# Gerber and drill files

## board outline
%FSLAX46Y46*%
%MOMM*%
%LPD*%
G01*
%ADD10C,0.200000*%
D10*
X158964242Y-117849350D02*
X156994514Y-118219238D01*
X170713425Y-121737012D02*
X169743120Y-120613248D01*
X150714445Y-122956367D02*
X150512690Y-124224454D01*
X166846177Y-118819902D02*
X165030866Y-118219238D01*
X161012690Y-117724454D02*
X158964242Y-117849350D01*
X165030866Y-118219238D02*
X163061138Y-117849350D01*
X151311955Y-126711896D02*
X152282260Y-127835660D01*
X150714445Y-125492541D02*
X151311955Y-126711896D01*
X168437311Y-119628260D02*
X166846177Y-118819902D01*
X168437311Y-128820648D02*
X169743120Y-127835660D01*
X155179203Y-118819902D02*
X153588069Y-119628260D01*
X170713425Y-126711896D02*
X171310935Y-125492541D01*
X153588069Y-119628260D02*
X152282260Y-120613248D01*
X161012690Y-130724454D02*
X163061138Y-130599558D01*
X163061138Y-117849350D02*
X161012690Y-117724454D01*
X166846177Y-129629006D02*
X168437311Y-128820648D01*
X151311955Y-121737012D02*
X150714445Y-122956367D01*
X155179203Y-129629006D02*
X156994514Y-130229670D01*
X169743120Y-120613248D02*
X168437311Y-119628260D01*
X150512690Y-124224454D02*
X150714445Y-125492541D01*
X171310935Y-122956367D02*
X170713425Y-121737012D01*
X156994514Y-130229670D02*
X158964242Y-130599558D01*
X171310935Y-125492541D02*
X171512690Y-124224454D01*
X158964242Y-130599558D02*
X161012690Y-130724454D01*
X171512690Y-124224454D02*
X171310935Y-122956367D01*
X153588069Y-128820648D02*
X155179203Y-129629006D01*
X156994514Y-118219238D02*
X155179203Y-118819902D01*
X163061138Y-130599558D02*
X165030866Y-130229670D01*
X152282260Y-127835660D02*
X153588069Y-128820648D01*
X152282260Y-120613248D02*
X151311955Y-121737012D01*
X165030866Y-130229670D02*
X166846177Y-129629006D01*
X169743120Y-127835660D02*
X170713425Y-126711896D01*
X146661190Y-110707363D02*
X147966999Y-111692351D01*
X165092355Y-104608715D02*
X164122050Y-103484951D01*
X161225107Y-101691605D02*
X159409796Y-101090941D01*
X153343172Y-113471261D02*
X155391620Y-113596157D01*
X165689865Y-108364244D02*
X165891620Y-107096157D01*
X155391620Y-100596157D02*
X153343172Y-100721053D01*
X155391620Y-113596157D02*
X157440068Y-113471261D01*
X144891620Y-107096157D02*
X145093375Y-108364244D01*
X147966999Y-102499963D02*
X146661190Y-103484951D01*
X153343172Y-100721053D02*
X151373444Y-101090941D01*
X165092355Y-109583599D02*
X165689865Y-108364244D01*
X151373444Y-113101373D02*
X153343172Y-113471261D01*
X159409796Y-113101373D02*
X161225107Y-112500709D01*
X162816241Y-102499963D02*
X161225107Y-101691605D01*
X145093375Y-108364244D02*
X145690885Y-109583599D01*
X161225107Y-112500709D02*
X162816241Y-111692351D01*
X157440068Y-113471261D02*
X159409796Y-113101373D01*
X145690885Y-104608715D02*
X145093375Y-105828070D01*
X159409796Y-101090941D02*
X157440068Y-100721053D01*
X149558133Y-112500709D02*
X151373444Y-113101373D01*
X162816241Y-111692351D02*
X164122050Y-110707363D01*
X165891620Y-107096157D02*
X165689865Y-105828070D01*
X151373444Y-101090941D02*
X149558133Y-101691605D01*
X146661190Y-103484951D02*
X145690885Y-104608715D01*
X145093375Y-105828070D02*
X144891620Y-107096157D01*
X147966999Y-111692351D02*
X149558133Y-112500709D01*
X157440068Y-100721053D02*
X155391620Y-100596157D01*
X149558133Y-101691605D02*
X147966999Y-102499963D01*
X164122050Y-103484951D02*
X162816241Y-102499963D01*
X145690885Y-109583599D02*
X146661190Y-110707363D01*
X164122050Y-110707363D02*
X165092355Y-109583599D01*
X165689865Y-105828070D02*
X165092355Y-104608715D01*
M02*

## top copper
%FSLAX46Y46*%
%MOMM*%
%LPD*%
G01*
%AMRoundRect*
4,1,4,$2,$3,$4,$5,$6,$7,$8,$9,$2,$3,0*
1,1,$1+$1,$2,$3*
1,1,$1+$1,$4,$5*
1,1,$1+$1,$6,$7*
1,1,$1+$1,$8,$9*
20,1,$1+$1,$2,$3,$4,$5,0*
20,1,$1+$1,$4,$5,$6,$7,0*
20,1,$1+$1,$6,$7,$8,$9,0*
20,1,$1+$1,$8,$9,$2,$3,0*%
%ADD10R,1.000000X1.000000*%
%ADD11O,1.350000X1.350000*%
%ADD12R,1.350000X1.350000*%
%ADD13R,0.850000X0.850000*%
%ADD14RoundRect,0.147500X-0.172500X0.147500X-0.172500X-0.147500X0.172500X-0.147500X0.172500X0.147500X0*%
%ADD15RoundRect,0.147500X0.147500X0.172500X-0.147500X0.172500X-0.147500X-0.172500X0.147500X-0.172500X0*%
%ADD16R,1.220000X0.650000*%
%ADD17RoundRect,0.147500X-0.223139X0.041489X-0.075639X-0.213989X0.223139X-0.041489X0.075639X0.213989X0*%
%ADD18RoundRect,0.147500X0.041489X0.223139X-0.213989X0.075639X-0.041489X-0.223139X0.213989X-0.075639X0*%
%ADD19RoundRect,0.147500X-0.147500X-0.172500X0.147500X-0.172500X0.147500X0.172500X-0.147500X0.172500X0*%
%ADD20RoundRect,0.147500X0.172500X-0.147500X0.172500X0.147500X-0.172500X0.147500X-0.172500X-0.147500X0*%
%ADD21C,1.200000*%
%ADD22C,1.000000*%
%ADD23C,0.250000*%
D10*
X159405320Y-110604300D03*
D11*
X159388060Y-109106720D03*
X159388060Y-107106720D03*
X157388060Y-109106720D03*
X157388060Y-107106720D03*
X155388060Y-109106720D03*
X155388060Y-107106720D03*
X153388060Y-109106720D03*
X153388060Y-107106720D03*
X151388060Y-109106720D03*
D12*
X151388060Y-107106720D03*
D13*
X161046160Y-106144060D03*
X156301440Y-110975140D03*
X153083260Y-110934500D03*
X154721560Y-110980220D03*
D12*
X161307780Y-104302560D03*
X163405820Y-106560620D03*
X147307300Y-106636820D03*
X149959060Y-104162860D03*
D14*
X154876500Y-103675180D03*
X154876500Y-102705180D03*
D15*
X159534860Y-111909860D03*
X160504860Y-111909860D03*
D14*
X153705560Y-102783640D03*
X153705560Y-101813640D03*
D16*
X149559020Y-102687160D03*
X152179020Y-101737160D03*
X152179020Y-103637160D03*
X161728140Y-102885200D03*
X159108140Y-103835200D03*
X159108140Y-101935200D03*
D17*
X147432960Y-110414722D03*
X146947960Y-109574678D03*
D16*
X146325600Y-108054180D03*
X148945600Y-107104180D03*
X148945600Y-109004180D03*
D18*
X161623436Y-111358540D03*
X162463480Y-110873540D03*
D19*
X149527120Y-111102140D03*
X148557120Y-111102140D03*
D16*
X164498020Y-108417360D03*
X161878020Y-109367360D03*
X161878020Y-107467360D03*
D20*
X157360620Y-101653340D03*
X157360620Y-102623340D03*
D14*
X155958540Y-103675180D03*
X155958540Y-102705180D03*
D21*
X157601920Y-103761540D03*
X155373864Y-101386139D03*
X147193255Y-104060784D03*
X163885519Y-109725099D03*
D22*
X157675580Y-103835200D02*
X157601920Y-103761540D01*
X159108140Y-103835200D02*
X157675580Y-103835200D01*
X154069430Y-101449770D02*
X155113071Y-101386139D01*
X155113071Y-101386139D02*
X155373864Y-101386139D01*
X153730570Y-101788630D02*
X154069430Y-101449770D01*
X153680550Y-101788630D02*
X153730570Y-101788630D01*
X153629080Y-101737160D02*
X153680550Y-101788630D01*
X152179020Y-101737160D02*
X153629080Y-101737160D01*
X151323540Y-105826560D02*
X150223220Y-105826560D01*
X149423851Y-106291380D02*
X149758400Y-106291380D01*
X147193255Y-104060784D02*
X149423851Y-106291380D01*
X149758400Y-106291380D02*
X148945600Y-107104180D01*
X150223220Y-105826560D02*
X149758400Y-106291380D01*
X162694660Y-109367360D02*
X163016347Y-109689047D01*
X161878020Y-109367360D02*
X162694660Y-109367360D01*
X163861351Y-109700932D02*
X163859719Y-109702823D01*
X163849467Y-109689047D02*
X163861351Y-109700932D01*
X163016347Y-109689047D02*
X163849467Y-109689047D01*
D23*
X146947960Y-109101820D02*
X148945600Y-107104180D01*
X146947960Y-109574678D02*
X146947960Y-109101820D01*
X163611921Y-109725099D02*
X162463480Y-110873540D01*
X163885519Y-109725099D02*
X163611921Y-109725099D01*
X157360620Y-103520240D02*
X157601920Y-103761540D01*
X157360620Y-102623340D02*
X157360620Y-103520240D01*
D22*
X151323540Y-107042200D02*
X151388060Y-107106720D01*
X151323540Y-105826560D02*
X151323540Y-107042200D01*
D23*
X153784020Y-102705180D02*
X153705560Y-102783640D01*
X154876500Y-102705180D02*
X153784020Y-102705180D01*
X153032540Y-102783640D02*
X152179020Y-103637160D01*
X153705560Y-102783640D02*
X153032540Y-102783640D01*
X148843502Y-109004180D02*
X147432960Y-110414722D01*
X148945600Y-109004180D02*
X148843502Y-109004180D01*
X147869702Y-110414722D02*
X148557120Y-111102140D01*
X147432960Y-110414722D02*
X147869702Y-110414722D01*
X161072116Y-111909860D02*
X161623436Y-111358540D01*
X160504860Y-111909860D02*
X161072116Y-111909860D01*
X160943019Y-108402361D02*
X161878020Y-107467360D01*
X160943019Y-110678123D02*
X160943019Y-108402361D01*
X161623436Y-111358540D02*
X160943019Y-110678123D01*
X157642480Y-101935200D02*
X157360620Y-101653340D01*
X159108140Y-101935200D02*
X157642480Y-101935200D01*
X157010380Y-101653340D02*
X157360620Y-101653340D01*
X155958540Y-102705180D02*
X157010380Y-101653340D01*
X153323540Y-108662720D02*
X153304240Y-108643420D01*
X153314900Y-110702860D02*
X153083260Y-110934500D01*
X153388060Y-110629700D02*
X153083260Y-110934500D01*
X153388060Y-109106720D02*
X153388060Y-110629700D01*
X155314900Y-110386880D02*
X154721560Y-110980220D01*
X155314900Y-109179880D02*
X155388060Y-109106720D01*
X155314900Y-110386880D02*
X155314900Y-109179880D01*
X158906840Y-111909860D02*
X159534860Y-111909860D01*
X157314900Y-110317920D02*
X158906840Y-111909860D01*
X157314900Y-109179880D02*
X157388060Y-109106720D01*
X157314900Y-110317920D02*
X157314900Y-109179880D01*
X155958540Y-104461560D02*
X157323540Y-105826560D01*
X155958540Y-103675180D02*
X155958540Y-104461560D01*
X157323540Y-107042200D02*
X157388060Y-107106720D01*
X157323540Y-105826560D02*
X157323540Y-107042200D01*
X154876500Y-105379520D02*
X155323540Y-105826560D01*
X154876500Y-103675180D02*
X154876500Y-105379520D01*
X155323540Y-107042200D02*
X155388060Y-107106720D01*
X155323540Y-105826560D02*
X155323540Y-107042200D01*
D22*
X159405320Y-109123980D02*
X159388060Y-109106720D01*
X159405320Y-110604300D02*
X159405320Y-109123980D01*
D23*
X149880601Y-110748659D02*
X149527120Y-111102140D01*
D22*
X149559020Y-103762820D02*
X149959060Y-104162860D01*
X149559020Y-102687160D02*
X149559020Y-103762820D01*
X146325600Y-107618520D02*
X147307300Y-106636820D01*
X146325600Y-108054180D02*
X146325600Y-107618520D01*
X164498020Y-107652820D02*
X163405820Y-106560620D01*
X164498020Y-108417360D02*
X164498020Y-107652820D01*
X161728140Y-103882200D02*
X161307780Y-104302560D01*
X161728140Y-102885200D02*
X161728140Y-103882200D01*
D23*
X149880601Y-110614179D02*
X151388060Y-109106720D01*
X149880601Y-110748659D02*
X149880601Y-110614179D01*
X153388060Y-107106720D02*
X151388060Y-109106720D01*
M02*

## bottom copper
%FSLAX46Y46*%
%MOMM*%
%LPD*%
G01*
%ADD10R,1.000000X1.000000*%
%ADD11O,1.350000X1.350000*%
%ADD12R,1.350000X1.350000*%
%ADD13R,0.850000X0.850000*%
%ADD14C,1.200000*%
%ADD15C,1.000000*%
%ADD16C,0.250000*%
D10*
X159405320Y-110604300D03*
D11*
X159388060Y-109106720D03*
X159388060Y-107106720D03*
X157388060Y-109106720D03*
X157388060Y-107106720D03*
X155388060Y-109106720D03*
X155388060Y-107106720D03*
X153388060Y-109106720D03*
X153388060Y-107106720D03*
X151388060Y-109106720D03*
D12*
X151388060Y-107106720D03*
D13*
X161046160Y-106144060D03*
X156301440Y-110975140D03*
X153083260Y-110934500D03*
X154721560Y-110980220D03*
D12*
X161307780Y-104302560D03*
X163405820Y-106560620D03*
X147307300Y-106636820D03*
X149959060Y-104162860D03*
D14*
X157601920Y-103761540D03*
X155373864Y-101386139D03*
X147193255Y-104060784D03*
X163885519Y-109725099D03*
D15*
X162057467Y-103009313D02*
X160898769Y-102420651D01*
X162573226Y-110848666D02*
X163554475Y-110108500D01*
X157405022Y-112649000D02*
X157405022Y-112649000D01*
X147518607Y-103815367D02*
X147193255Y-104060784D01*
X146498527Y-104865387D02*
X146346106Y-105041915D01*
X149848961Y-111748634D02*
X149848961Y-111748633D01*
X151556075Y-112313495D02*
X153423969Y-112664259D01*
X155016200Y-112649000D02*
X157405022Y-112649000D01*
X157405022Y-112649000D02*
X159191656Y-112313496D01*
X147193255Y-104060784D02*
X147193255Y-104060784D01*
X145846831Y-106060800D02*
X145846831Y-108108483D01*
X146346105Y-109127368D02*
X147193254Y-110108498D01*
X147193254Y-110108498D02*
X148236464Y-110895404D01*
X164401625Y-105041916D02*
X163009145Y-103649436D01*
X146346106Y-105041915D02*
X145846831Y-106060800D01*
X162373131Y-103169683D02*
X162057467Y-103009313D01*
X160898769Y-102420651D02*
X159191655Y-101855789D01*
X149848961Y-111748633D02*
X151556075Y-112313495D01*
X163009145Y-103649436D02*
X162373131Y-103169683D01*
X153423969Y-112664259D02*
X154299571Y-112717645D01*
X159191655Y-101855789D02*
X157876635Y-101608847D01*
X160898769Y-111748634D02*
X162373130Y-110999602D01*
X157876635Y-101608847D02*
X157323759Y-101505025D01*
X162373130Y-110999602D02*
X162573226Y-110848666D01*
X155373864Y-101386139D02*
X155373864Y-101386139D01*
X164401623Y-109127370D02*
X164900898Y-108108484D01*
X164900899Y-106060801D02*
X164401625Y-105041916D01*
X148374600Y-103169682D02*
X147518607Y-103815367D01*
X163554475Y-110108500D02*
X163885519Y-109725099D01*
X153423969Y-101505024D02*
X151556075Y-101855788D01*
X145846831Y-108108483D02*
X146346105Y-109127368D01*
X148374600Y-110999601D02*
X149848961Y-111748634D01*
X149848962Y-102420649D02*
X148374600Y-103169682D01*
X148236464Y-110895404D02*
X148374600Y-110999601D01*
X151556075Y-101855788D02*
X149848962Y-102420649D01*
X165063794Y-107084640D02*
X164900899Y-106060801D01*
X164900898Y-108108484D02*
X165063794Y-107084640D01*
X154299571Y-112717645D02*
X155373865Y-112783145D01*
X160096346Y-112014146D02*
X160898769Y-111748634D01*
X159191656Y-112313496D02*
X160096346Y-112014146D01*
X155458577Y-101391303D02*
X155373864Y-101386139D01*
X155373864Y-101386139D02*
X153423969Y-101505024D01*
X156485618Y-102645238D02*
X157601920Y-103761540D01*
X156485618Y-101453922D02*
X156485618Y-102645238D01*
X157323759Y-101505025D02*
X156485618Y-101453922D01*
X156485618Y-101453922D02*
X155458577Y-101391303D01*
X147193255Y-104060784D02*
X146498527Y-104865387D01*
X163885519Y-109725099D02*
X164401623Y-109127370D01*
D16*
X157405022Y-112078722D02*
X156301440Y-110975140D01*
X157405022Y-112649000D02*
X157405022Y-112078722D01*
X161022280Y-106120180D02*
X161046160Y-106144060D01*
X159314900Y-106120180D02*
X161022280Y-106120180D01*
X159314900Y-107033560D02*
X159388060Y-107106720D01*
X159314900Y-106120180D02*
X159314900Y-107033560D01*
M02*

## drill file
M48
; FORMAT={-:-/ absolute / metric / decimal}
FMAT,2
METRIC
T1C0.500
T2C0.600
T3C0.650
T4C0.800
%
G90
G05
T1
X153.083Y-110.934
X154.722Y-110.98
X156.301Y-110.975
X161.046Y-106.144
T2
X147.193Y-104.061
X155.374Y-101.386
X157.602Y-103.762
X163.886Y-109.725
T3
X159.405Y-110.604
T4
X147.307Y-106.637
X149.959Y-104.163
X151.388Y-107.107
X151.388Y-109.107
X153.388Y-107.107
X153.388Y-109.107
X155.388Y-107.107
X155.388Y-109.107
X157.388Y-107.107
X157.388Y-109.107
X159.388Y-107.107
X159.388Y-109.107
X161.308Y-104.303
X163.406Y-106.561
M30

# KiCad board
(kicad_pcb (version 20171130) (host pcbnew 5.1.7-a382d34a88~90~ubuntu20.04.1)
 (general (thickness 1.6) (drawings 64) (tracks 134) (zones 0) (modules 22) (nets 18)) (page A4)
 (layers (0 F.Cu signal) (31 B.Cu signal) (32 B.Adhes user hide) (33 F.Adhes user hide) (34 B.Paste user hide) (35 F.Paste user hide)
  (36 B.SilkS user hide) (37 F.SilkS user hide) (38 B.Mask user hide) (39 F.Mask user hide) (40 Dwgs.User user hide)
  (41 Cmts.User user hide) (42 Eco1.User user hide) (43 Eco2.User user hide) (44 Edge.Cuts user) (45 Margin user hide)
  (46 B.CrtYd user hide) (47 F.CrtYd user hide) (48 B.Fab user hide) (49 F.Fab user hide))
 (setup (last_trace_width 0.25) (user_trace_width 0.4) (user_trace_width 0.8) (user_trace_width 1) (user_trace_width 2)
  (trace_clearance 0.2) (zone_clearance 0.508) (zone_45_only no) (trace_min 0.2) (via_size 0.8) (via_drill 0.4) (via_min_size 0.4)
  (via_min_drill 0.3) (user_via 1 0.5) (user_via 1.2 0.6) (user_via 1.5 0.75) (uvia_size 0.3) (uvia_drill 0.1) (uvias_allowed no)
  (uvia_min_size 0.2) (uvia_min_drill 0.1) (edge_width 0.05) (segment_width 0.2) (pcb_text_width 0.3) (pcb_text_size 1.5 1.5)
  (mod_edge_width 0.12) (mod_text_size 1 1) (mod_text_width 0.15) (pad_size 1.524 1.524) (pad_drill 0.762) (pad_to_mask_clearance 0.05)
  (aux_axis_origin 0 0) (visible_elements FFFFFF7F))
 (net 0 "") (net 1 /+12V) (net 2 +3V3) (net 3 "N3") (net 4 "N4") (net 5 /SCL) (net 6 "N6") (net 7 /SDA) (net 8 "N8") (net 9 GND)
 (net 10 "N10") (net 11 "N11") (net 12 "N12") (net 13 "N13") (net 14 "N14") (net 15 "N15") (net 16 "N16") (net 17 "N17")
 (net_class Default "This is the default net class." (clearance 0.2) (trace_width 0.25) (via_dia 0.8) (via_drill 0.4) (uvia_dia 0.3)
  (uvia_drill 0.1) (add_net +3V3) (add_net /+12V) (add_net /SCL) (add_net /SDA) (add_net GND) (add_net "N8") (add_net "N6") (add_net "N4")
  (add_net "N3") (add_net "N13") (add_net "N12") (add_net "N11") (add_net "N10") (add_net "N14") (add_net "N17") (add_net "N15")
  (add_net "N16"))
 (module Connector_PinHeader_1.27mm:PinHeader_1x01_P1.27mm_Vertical (layer F.Cu) (at 159.40532 110.6043)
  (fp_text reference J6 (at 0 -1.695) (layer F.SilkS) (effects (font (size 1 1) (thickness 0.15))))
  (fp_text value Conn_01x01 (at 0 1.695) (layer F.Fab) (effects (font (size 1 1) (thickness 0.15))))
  (pad 1 thru_hole rect (at 0 0) (size 1 1) (drill 0.65) (layers *.Cu *.Mask) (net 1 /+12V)))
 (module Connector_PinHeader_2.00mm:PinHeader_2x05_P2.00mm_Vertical (layer B.Cu) (at 151.38806 107.10672 270)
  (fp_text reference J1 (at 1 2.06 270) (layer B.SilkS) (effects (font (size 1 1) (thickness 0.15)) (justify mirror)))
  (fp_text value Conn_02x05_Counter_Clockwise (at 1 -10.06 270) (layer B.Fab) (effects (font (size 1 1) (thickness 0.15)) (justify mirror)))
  (pad 10 thru_hole oval (at 2 -8 270) (size 1.35 1.35) (drill 0.8) (layers *.Cu *.Mask) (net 1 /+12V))
  (pad 9 thru_hole oval (at 0 -8 270) (size 1.35 1.35) (drill 0.8) (layers *.Cu *.Mask) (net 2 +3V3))
  (pad 8 thru_hole oval (at 2 -6 270) (size 1.35 1.35) (drill 0.8) (layers *.Cu *.Mask) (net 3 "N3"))
  (pad 7 thru_hole oval (at 0 -6 270) (size 1.35 1.35) (drill 0.8) (layers *.Cu *.Mask) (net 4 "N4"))
  (pad 6 thru_hole oval (at 2 -4 270) (size 1.35 1.35) (drill 0.8) (layers *.Cu *.Mask) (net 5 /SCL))
  (pad 5 thru_hole oval (at 0 -4 270) (size 1.35 1.35) (drill 0.8) (layers *.Cu *.Mask) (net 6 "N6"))
  (pad 4 thru_hole oval (at 2 -2 270) (size 1.35 1.35) (drill 0.8) (layers *.Cu *.Mask) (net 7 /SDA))
  (pad 3 thru_hole oval (at 0 -2 270) (size 1.35 1.35) (drill 0.8) (layers *.Cu *.Mask) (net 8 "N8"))
  (pad 2 thru_hole oval (at 2 0 270) (size 1.35 1.35) (drill 0.8) (layers *.Cu *.Mask) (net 8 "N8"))
  (pad 1 thru_hole rect (at 0 0 270) (size 1.35 1.35) (drill 0.8) (layers *.Cu *.Mask) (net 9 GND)))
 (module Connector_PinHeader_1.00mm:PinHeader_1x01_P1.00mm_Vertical (layer F.Cu) (at 161.04616 106.14406)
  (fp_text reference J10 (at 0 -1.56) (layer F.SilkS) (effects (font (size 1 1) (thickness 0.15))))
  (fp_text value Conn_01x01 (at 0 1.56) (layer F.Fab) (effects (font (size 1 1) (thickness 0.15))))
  (pad 1 thru_hole rect (at 0 0) (size 0.85 0.85) (drill 0.5) (layers *.Cu *.Mask) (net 2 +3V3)))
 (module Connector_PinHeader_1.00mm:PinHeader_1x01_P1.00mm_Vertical (layer F.Cu) (at 156.30144 110.97514)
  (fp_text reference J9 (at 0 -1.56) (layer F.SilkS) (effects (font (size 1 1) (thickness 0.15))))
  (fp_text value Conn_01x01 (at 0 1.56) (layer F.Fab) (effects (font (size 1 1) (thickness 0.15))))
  (pad 1 thru_hole rect (at 0 0) (size 0.85 0.85) (drill 0.5) (layers *.Cu *.Mask) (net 9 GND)))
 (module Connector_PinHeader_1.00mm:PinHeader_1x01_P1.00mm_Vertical (layer F.Cu) (at 153.08326 110.9345)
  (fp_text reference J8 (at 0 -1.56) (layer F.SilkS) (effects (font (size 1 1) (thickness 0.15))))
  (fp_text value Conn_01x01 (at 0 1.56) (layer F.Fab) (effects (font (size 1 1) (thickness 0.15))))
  (pad 1 thru_hole rect (at 0 0) (size 0.85 0.85) (drill 0.5) (layers *.Cu *.Mask) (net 7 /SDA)))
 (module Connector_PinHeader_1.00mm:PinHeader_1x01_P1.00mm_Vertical (layer F.Cu) (at 154.72156 110.98022)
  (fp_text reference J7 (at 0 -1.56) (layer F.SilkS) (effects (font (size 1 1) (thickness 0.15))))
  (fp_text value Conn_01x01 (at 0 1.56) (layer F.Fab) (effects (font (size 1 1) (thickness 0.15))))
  (pad 1 thru_hole rect (at 0 0) (size 0.85 0.85) (drill 0.5) (layers *.Cu *.Mask) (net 5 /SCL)))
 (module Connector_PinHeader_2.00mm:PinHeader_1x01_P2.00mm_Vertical (layer F.Cu) (at 161.30778 104.30256)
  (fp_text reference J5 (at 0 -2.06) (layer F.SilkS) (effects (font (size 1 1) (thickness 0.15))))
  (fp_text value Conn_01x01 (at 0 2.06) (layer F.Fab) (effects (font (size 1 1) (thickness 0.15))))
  (pad 1 thru_hole rect (at 0 0) (size 1.35 1.35) (drill 0.8) (layers *.Cu *.Mask) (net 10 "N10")))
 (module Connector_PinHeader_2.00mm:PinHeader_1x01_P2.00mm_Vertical (layer F.Cu) (at 163.40582 106.56062)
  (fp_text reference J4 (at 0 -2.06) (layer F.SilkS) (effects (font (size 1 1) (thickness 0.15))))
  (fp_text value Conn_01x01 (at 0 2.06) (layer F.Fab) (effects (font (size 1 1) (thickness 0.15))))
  (pad 1 thru_hole rect (at 0 0) (size 1.35 1.35) (drill 0.8) (layers *.Cu *.Mask) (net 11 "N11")))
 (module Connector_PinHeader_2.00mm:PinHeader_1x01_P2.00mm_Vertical (layer F.Cu) (at 147.3073 106.63682)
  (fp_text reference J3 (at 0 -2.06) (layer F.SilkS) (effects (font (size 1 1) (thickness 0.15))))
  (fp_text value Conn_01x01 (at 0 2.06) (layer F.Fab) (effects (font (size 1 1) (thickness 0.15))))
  (pad 1 thru_hole rect (at 0 0) (size 1.35 1.35) (drill 0.8) (layers *.Cu *.Mask) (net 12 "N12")))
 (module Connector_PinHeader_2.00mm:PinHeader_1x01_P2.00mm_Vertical (layer F.Cu) (at 149.95906 104.16286)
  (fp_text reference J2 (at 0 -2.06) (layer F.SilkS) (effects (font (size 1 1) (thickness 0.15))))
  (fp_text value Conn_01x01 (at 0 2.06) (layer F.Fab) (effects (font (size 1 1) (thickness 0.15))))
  (pad 1 thru_hole rect (at 0 0) (size 1.35 1.35) (drill 0.8) (layers *.Cu *.Mask) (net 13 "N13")))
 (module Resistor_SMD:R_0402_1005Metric (layer F.Cu) (at 154.8765 103.19018 270)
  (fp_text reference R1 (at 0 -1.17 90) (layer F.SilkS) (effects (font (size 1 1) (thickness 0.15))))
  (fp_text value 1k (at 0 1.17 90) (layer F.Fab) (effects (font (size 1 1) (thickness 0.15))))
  (pad 2 smd roundrect (at 0.485 0 270) (size 0.59 0.64) (layers F.Cu F.Paste F.Mask) (roundrect_rratio 0.25) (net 6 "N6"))
  (pad 1 smd roundrect (at -0.485 0 270) (size 0.59 0.64) (layers F.Cu F.Paste F.Mask) (roundrect_rratio 0.25) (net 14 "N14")))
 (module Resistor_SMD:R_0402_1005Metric (layer F.Cu) (at 160.01986 111.90986 180)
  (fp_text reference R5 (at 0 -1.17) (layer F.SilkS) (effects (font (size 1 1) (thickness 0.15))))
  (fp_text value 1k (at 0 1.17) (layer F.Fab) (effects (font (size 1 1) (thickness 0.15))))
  (pad 2 smd roundrect (at 0.485 0 180) (size 0.59 0.64) (layers F.Cu F.Paste F.Mask) (roundrect_rratio 0.25) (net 3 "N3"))
  (pad 1 smd roundrect (at -0.485 0 180) (size 0.59 0.64) (layers F.Cu F.Paste F.Mask) (roundrect_rratio 0.25) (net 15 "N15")))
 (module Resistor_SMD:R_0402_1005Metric (layer F.Cu) (at 153.70556 102.29864 270)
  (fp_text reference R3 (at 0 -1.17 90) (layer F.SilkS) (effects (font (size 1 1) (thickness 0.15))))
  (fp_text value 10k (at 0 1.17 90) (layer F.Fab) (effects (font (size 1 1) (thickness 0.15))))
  (pad 2 smd roundrect (at 0.485 0 270) (size 0.59 0.64) (layers F.Cu F.Paste F.Mask) (roundrect_rratio 0.25) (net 14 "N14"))
  (pad 1 smd roundrect (at -0.485 0 270) (size 0.59 0.64) (layers F.Cu F.Paste F.Mask) (roundrect_rratio 0.25) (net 9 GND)))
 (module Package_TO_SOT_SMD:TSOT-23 (layer F.Cu) (at 150.86902 102.68716 180)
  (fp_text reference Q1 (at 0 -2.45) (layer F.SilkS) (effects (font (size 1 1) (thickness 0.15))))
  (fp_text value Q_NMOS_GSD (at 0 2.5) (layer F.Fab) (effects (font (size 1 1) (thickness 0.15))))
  (pad 3 smd rect (at 1.31 0 180) (size 1.22 0.65) (layers F.Cu F.Paste F.Mask) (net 13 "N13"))
  (pad 2 smd rect (at -1.31 0.95 180) (size 1.22 0.65) (layers F.Cu F.Paste F.Mask) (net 9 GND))
  (pad 1 smd rect (at -1.31 -0.95 180) (size 1.22 0.65) (layers F.Cu F.Paste F.Mask) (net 14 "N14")))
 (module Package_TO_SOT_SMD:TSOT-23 (layer F.Cu) (at 160.41814 102.8852)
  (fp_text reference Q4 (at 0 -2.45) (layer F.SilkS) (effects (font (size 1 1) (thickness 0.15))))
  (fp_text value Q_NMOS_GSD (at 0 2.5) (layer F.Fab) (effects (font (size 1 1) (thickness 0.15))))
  (pad 3 smd rect (at 1.31 0) (size 1.22 0.65) (layers F.Cu F.Paste F.Mask) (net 10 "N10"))
  (pad 2 smd rect (at -1.31 0.95) (size 1.22 0.65) (layers F.Cu F.Paste F.Mask) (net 9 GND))
  (pad 1 smd rect (at -1.31 -0.95) (size 1.22 0.65) (layers F.Cu F.Paste F.Mask) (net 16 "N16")))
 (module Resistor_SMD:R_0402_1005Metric (layer F.Cu) (at 147.19046 109.9947 300)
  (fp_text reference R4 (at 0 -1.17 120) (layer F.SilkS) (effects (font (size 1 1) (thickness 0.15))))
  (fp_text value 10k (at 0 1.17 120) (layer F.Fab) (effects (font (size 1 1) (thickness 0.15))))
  (pad 2 smd roundrect (at 0.485 0 300) (size 0.59 0.64) (layers F.Cu F.Paste F.Mask) (roundrect_rratio 0.25) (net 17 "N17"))
  (pad 1 smd roundrect (at -0.485 0 300) (size 0.59 0.64) (layers F.Cu F.Paste F.Mask) (roundrect_rratio 0.25) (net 9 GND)))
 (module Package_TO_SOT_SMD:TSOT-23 (layer F.Cu) (at 147.6356 108.05418 180)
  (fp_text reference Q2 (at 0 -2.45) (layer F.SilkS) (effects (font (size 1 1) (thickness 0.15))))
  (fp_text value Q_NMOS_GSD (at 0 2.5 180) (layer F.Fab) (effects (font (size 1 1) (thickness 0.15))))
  (pad 3 smd rect (at 1.31 0 180) (size 1.22 0.65) (layers F.Cu F.Paste F.Mask) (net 12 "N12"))
  (pad 2 smd rect (at -1.31 0.95 180) (size 1.22 0.65) (layers F.Cu F.Paste F.Mask) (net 9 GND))
  (pad 1 smd rect (at -1.31 -0.95 180) (size 1.22 0.65) (layers F.Cu F.Paste F.Mask) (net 17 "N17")))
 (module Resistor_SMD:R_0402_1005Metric (layer F.Cu) (at 162.043458 111.11604 210)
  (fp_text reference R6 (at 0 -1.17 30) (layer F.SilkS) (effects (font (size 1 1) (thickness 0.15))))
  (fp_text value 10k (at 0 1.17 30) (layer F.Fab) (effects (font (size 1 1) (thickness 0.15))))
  (pad 2 smd roundrect (at 0.485 0 210) (size 0.59 0.64) (layers F.Cu F.Paste F.Mask) (roundrect_rratio 0.25) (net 15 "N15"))
  (pad 1 smd roundrect (at -0.485 0 210) (size 0.59 0.64) (layers F.Cu F.Paste F.Mask) (roundrect_rratio 0.25) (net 9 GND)))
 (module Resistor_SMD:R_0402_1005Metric (layer F.Cu) (at 149.04212 111.10214)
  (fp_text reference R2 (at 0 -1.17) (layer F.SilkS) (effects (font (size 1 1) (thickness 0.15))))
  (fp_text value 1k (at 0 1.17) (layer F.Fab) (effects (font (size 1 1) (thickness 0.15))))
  (pad 2 smd roundrect (at 0.485 0) (size 0.59 0.64) (layers F.Cu F.Paste F.Mask) (roundrect_rratio 0.25) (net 8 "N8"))
  (pad 1 smd roundrect (at -0.485 0) (size 0.59 0.64) (layers F.Cu F.Paste F.Mask) (roundrect_rratio 0.25) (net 17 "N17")))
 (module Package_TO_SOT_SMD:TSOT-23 (layer F.Cu) (at 163.18802 108.41736)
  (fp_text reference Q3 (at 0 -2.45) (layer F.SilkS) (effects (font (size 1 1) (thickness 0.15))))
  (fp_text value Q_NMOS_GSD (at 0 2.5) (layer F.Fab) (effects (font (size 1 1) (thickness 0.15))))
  (pad 3 smd rect (at 1.31 0) (size 1.22 0.65) (layers F.Cu F.Paste F.Mask) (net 11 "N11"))
  (pad 2 smd rect (at -1.31 0.95) (size 1.22 0.65) (layers F.Cu F.Paste F.Mask) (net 9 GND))
  (pad 1 smd rect (at -1.31 -0.95) (size 1.22 0.65) (layers F.Cu F.Paste F.Mask) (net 15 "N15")))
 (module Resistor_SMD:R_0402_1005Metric (layer F.Cu) (at 157.36062 102.13834 90)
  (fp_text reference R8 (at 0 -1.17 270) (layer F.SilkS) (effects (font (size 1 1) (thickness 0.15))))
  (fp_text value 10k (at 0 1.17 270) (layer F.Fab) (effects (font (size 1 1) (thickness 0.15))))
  (pad 2 smd roundrect (at 0.485 0 90) (size 0.59 0.64) (layers F.Cu F.Paste F.Mask) (roundrect_rratio 0.25) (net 16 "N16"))
  (pad 1 smd roundrect (at -0.485 0 90) (size 0.59 0.64) (layers F.Cu F.Paste F.Mask) (roundrect_rratio 0.25) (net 9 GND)))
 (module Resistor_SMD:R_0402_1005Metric (layer F.Cu) (at 155.95854 103.19018 270)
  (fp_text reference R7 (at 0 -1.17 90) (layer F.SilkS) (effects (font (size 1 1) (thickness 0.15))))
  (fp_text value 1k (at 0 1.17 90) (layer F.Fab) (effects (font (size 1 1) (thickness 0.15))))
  (pad 2 smd roundrect (at 0.485 0 270) (size 0.59 0.64) (layers F.Cu F.Paste F.Mask) (roundrect_rratio 0.25) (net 4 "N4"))
  (pad 1 smd roundrect (at -0.485 0 270) (size 0.59 0.64) (layers F.Cu F.Paste F.Mask) (roundrect_rratio 0.25) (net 16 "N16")))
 (gr_line (start 158.964242 117.84935) (end 156.994514 118.219238) (layer Edge.Cuts) (width 0.2))
 (gr_line (start 170.713425 121.737012) (end 169.74312 120.613248) (layer Edge.Cuts) (width 0.2))
 (gr_line (start 150.714445 122.956367) (end 150.51269 124.224454) (layer Edge.Cuts) (width 0.2))
 (gr_line (start 166.846177 118.819902) (end 165.030866 118.219238) (layer Edge.Cuts) (width 0.2))
 (gr_line (start 161.01269 117.724454) (end 158.964242 117.84935) (layer Edge.Cuts) (width 0.2))
 (gr_line (start 165.030866 118.219238) (end 163.061138 117.84935) (layer Edge.Cuts) (width 0.2))
 (gr_line (start 151.311955 126.711896) (end 152.28226 127.83566) (layer Edge.Cuts) (width 0.2))
 (gr_line (start 150.714445 125.492541) (end 151.311955 126.711896) (layer Edge.Cuts) (width 0.2))
 (gr_line (start 168.437311 119.62826) (end 166.846177 118.819902) (layer Edge.Cuts) (width 0.2))
 (gr_line (start 168.437311 128.820648) (end 169.74312 127.83566) (layer Edge.Cuts) (width 0.2))
 (gr_line (start 155.179203 118.819902) (end 153.588069 119.62826) (layer Edge.Cuts) (width 0.2))
 (gr_line (start 170.713425 126.711896) (end 171.310935 125.492541) (layer Edge.Cuts) (width 0.2))
 (gr_line (start 153.588069 119.62826) (end 152.28226 120.613248) (layer Edge.Cuts) (width 0.2))
 (gr_line (start 161.01269 130.724454) (end 163.061138 130.599558) (layer Edge.Cuts) (width 0.2))
 (gr_line (start 163.061138 117.84935) (end 161.01269 117.724454) (layer Edge.Cuts) (width 0.2))
 (gr_line (start 166.846177 129.629006) (end 168.437311 128.820648) (layer Edge.Cuts) (width 0.2))
 (gr_line (start 151.311955 121.737012) (end 150.714445 122.956367) (layer Edge.Cuts) (width 0.2))
 (gr_line (start 155.179203 129.629006) (end 156.994514 130.22967) (layer Edge.Cuts) (width 0.2))
 (gr_line (start 169.74312 120.613248) (end 168.437311 119.62826) (layer Edge.Cuts) (width 0.2))
 (gr_line (start 150.51269 124.224454) (end 150.714445 125.492541) (layer Edge.Cuts) (width 0.2))
 (gr_line (start 171.310935 122.956367) (end 170.713425 121.737012) (layer Edge.Cuts) (width 0.2))
 (gr_line (start 156.994514 130.22967) (end 158.964242 130.599558) (layer Edge.Cuts) (width 0.2))
 (gr_line (start 171.310935 125.492541) (end 171.51269 124.224454) (layer Edge.Cuts) (width 0.2))
 (gr_line (start 158.964242 130.599558) (end 161.01269 130.724454) (layer Edge.Cuts) (width 0.2))
 (gr_line (start 171.51269 124.224454) (end 171.310935 122.956367) (layer Edge.Cuts) (width 0.2))
 (gr_line (start 153.588069 128.820648) (end 155.179203 129.629006) (layer Edge.Cuts) (width 0.2))
 (gr_line (start 156.994514 118.219238) (end 155.179203 118.819902) (layer Edge.Cuts) (width 0.2))
 (gr_line (start 163.061138 130.599558) (end 165.030866 130.22967) (layer Edge.Cuts) (width 0.2))
 (gr_line (start 152.28226 127.83566) (end 153.588069 128.820648) (layer Edge.Cuts) (width 0.2))
 (gr_line (start 152.28226 120.613248) (end 151.311955 121.737012) (layer Edge.Cuts) (width 0.2))
 (gr_line (start 165.030866 130.22967) (end 166.846177 129.629006) (layer Edge.Cuts) (width 0.2))
 (gr_line (start 169.74312 127.83566) (end 170.713425 126.711896) (layer Edge.Cuts) (width 0.2))
 (gr_line (start 146.66119 110.707363) (end 147.966999 111.692351) (layer Edge.Cuts) (width 0.2))
 (gr_line (start 165.092355 104.608715) (end 164.12205 103.484951) (layer Edge.Cuts) (width 0.2))
 (gr_line (start 161.225107 101.691605) (end 159.409796 101.090941) (layer Edge.Cuts) (width 0.2))
 (gr_line (start 153.343172 113.471261) (end 155.39162 113.596157) (layer Edge.Cuts) (width 0.2))
 (gr_line (start 165.689865 108.364244) (end 165.89162 107.096157) (layer Edge.Cuts) (width 0.2))
 (gr_line (start 155.39162 100.596157) (end 153.343172 100.721053) (layer Edge.Cuts) (width 0.2))
 (gr_line (start 155.39162 113.596157) (end 157.440068 113.471261) (layer Edge.Cuts) (width 0.2))
 (gr_line (start 144.89162 107.096157) (end 145.093375 108.364244) (layer Edge.Cuts) (width 0.2))
 (gr_line (start 147.966999 102.499963) (end 146.66119 103.484951) (layer Edge.Cuts) (width 0.2))
 (gr_line (start 153.343172 100.721053) (end 151.373444 101.090941) (layer Edge.Cuts) (width 0.2))
 (gr_line (start 165.092355 109.583599) (end 165.689865 108.364244) (layer Edge.Cuts) (width 0.2))
 (gr_line (start 151.373444 113.101373) (end 153.343172 113.471261) (layer Edge.Cuts) (width 0.2))
 (gr_line (start 159.409796 113.101373) (end 161.225107 112.500709) (layer Edge.Cuts) (width 0.2))
 (gr_line (start 162.816241 102.499963) (end 161.225107 101.691605) (layer Edge.Cuts) (width 0.2))
 (gr_line (start 145.093375 108.364244) (end 145.690885 109.583599) (layer Edge.Cuts) (width 0.2))
 (gr_line (start 161.225107 112.500709) (end 162.816241 111.692351) (layer Edge.Cuts) (width 0.2))
 (gr_line (start 157.440068 113.471261) (end 159.409796 113.101373) (layer Edge.Cuts) (width 0.2))
 (gr_line (start 145.690885 104.608715) (end 145.093375 105.82807) (layer Edge.Cuts) (width 0.2))
 (gr_line (start 159.409796 101.090941) (end 157.440068 100.721053) (layer Edge.Cuts) (width 0.2))
 (gr_line (start 149.558133 112.500709) (end 151.373444 113.101373) (layer Edge.Cuts) (width 0.2))
 (gr_line (start 162.816241 111.692351) (end 164.12205 110.707363) (layer Edge.Cuts) (width 0.2))
 (gr_line (start 165.89162 107.096157) (end 165.689865 105.82807) (layer Edge.Cuts) (width 0.2))
 (gr_line (start 151.373444 101.090941) (end 149.558133 101.691605) (layer Edge.Cuts) (width 0.2))
 (gr_line (start 146.66119 103.484951) (end 145.690885 104.608715) (layer Edge.Cuts) (width 0.2))
 (gr_line (start 145.093375 105.82807) (end 144.89162 107.096157) (layer Edge.Cuts) (width 0.2))
 (gr_line (start 147.966999 111.692351) (end 149.558133 112.500709) (layer Edge.Cuts) (width 0.2))
 (gr_line (start 157.440068 100.721053) (end 155.39162 100.596157) (layer Edge.Cuts) (width 0.2))
 (gr_line (start 149.558133 101.691605) (end 147.966999 102.499963) (layer Edge.Cuts) (width 0.2))
 (gr_line (start 164.12205 103.484951) (end 162.816241 102.499963) (layer Edge.Cuts) (width 0.2))
 (gr_line (start 145.690885 109.583599) (end 146.66119 110.707363) (layer Edge.Cuts) (width 0.2))
 (gr_line (start 164.12205 110.707363) (end 165.092355 109.583599) (layer Edge.Cuts) (width 0.2))
 (gr_line (start 165.689865 105.82807) (end 165.092355 104.608715) (layer Edge.Cuts) (width 0.2))
 (segment (start 162.057467 103.009313) (end 160.898769 102.420651) (width 1) (layer B.Cu) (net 9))
 (segment (start 162.573226 110.848666) (end 163.554475 110.1085) (width 1) (layer B.Cu) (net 9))
 (segment (start 157.405022 112.649) (end 157.405022 112.649) (width 1) (layer B.Cu) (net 9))
 (segment (start 147.518607 103.815367) (end 147.193255 104.060784) (width 1) (layer B.Cu) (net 9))
 (segment (start 146.498527 104.865387) (end 146.346106 105.041915) (width 1) (layer B.Cu) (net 9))
 (segment (start 149.848961 111.748634) (end 149.848961 111.748633) (width 1) (layer B.Cu) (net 9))
 (segment (start 151.556075 112.313495) (end 153.423969 112.664259) (width 1) (layer B.Cu) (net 9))
 (segment (start 155.0162 112.649) (end 157.405022 112.649) (width 1) (layer B.Cu) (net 9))
 (segment (start 157.405022 112.649) (end 159.191656 112.313496) (width 1) (layer B.Cu) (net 9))
 (segment (start 147.193255 104.060784) (end 147.193255 104.060784) (width 1) (layer B.Cu) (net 9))
 (segment (start 145.846831 106.0608) (end 145.846831 108.108483) (width 1) (layer B.Cu) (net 9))
 (segment (start 146.346105 109.127368) (end 147.193254 110.108498) (width 1) (layer B.Cu) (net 9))
 (segment (start 147.193254 110.108498) (end 148.236464 110.895404) (width 1) (layer B.Cu) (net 9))
 (segment (start 164.401625 105.041916) (end 163.009145 103.649436) (width 1) (layer B.Cu) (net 9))
 (segment (start 146.346106 105.041915) (end 145.846831 106.0608) (width 1) (layer B.Cu) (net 9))
 (segment (start 162.373131 103.169683) (end 162.057467 103.009313) (width 1) (layer B.Cu) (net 9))
 (segment (start 160.898769 102.420651) (end 159.191655 101.855789) (width 1) (layer B.Cu) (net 9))
 (segment (start 149.848961 111.748633) (end 151.556075 112.313495) (width 1) (layer B.Cu) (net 9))
 (segment (start 163.009145 103.649436) (end 162.373131 103.169683) (width 1) (layer B.Cu) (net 9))
 (segment (start 153.423969 112.664259) (end 154.299571 112.717645) (width 1) (layer B.Cu) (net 9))
 (segment (start 159.191655 101.855789) (end 157.876635 101.608847) (width 1) (layer B.Cu) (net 9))
 (segment (start 160.898769 111.748634) (end 162.37313 110.999602) (width 1) (layer B.Cu) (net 9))
 (segment (start 157.876635 101.608847) (end 157.323759 101.505025) (width 1) (layer B.Cu) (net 9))
 (segment (start 162.37313 110.999602) (end 162.573226 110.848666) (width 1) (layer B.Cu) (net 9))
 (segment (start 155.373864 101.386139) (end 155.373864 101.386139) (width 1) (layer B.Cu) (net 9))
 (segment (start 164.401623 109.12737) (end 164.900898 108.108484) (width 1) (layer B.Cu) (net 9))
 (segment (start 164.900899 106.060801) (end 164.401625 105.041916) (width 1) (layer B.Cu) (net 9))
 (segment (start 148.3746 103.169682) (end 147.518607 103.815367) (width 1) (layer B.Cu) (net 9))
 (segment (start 163.554475 110.1085) (end 163.885519 109.725099) (width 1) (layer B.Cu) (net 9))
 (segment (start 153.423969 101.505024) (end 151.556075 101.855788) (width 1) (layer B.Cu) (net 9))
 (segment (start 145.846831 108.108483) (end 146.346105 109.127368) (width 1) (layer B.Cu) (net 9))
 (segment (start 148.3746 110.999601) (end 149.848961 111.748634) (width 1) (layer B.Cu) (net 9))
 (segment (start 149.848962 102.420649) (end 148.3746 103.169682) (width 1) (layer B.Cu) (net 9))
 (segment (start 148.236464 110.895404) (end 148.3746 110.999601) (width 1) (layer B.Cu) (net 9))
 (segment (start 151.556075 101.855788) (end 149.848962 102.420649) (width 1) (layer B.Cu) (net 9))
 (segment (start 165.063794 107.08464) (end 164.900899 106.060801) (width 1) (layer B.Cu) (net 9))
 (segment (start 164.900898 108.108484) (end 165.063794 107.08464) (width 1) (layer B.Cu) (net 9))
 (segment (start 154.299571 112.717645) (end 155.373865 112.783145) (width 1) (layer B.Cu) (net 9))
 (segment (start 160.096346 112.014146) (end 160.898769 111.748634) (width 1) (layer B.Cu) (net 9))
 (segment (start 159.191656 112.313496) (end 160.096346 112.014146) (width 1) (layer B.Cu) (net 9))
 (segment (start 155.458577 101.391303) (end 155.373864 101.386139) (width 1) (layer B.Cu) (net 9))
 (via (at 157.60192 103.76154) (size 1.2) (drill 0.6) (layers F.Cu B.Cu) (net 9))
 (segment (start 155.373864 101.386139) (end 153.423969 101.505024) (width 1) (layer B.Cu) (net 9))
 (via (at 155.373864 101.386139) (size 1.2) (drill 0.6) (layers F.Cu B.Cu) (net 9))
 (segment (start 156.485618 102.645238) (end 157.60192 103.76154) (width 1) (layer B.Cu) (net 9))
 (segment (start 156.485618 101.453922) (end 156.485618 102.645238) (width 1) (layer B.Cu) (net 9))
 (segment (start 157.323759 101.505025) (end 156.485618 101.453922) (width 1) (layer B.Cu) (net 9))
 (segment (start 156.485618 101.453922) (end 155.458577 101.391303) (width 1) (layer B.Cu) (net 9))
 (segment (start 157.67558 103.8352) (end 157.60192 103.76154) (width 1) (layer F.Cu) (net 9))
 (segment (start 159.10814 103.8352) (end 157.67558 103.8352) (width 1) (layer F.Cu) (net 9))
 (segment (start 154.06943 101.44977) (end 155.113071 101.386139) (width 1) (layer F.Cu) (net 9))
 (segment (start 155.113071 101.386139) (end 155.373864 101.386139) (width 1) (layer F.Cu) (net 9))
 (segment (start 153.73057 101.78863) (end 154.06943 101.44977) (width 1) (layer F.Cu) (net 9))
 (segment (start 153.68055 101.78863) (end 153.73057 101.78863) (width 1) (layer F.Cu) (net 9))
 (segment (start 153.62908 101.73716) (end 153.68055 101.78863) (width 1) (layer F.Cu) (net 9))
 (segment (start 152.17902 101.73716) (end 153.62908 101.73716) (width 1) (layer F.Cu) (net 9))
 (segment (start 151.32354 105.82656) (end 150.22322 105.82656) (width 1) (layer F.Cu) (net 9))
 (segment (start 147.193255 104.060784) (end 146.498527 104.865387) (width 1) (layer B.Cu) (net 9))
 (via (at 147.193255 104.060784) (size 1.2) (drill 0.6) (layers F.Cu B.Cu) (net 9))
 (segment (start 149.423851 106.29138) (end 149.7584 106.29138) (width 1) (layer F.Cu) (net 9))
 (segment (start 147.193255 104.060784) (end 149.423851 106.29138) (width 1) (layer F.Cu) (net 9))
 (segment (start 149.7584 106.29138) (end 148.9456 107.10418) (width 1) (layer F.Cu) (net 9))
 (segment (start 150.22322 105.82656) (end 149.7584 106.29138) (width 1) (layer F.Cu) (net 9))
 (segment (start 163.885519 109.725099) (end 164.401623 109.12737) (width 1) (layer B.Cu) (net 9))
 (via (at 163.885519 109.725099) (size 1.2) (drill 0.6) (layers F.Cu B.Cu) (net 9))
 (segment (start 162.69466 109.36736) (end 163.016347 109.689047) (width 1) (layer F.Cu) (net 9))
 (segment (start 161.87802 109.36736) (end 162.69466 109.36736) (width 1) (layer F.Cu) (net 9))
 (segment (start 163.861351 109.700932) (end 163.859719 109.702823) (width 1) (layer F.Cu) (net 9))
 (segment (start 163.849467 109.689047) (end 163.861351 109.700932) (width 1) (layer F.Cu) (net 9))
 (segment (start 163.016347 109.689047) (end 163.849467 109.689047) (width 1) (layer F.Cu) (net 9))
 (segment (start 146.94796 109.10182) (end 148.9456 107.10418) (width 0.25) (layer F.Cu) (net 9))
 (segment (start 146.94796 109.574678) (end 146.94796 109.10182) (width 0.25) (layer F.Cu) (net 9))
 (segment (start 163.611921 109.725099) (end 162.46348 110.87354) (width 0.25) (layer F.Cu) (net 9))
 (segment (start 163.885519 109.725099) (end 163.611921 109.725099) (width 0.25) (layer F.Cu) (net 9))
 (segment (start 157.36062 103.52024) (end 157.60192 103.76154) (width 0.25) (layer F.Cu) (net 9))
 (segment (start 157.36062 102.62334) (end 157.36062 103.52024) (width 0.25) (layer F.Cu) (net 9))
 (segment (start 157.405022 112.078722) (end 156.30144 110.97514) (width 0.25) (layer B.Cu) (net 9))
 (segment (start 157.405022 112.649) (end 157.405022 112.078722) (width 0.25) (layer B.Cu) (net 9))
 (segment (start 151.32354 107.0422) (end 151.38806 107.10672) (width 1) (layer F.Cu) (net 9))
 (segment (start 151.32354 105.82656) (end 151.32354 107.0422) (width 1) (layer F.Cu) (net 9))
 (segment (start 153.78402 102.70518) (end 153.70556 102.78364) (width 0.25) (layer F.Cu) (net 14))
 (segment (start 154.8765 102.70518) (end 153.78402 102.70518) (width 0.25) (layer F.Cu) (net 14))
 (segment (start 153.03254 102.78364) (end 152.17902 103.63716) (width 0.25) (layer F.Cu) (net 14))
 (segment (start 153.70556 102.78364) (end 153.03254 102.78364) (width 0.25) (layer F.Cu) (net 14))
 (segment (start 148.843502 109.00418) (end 147.43296 110.414722) (width 0.25) (layer F.Cu) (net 17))
 (segment (start 148.9456 109.00418) (end 148.843502 109.00418) (width 0.25) (layer F.Cu) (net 17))
 (segment (start 147.869702 110.414722) (end 148.55712 111.10214) (width 0.25) (layer F.Cu) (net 17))
 (segment (start 147.43296 110.414722) (end 147.869702 110.414722) (width 0.25) (layer F.Cu) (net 17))
 (segment (start 161.072116 111.90986) (end 161.623436 111.35854) (width 0.25) (layer F.Cu) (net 15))
 (segment (start 160.50486 111.90986) (end 161.072116 111.90986) (width 0.25) (layer F.Cu) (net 15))
 (segment (start 160.943019 108.402361) (end 161.87802 107.46736) (width 0.25) (layer F.Cu) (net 15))
 (segment (start 160.943019 110.678123) (end 160.943019 108.402361) (width 0.25) (layer F.Cu) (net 15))
 (segment (start 161.623436 111.35854) (end 160.943019 110.678123) (width 0.25) (layer F.Cu) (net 15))
 (segment (start 157.64248 101.9352) (end 157.36062 101.65334) (width 0.25) (layer F.Cu) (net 16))
 (segment (start 159.10814 101.9352) (end 157.64248 101.9352) (width 0.25) (layer F.Cu) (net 16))
 (segment (start 157.01038 101.65334) (end 157.36062 101.65334) (width 0.25) (layer F.Cu) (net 16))
 (segment (start 155.95854 102.70518) (end 157.01038 101.65334) (width 0.25) (layer F.Cu) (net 16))
 (segment (start 153.32354 108.66272) (end 153.30424 108.64342) (width 0.25) (layer F.Cu) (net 7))
 (segment (start 153.3149 110.70286) (end 153.08326 110.9345) (width 0.25) (layer F.Cu) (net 7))
 (segment (start 153.38806 110.6297) (end 153.08326 110.9345) (width 0.25) (layer F.Cu) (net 7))
 (segment (start 153.38806 109.10672) (end 153.38806 110.6297) (width 0.25) (layer F.Cu) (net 7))
 (segment (start 155.3149 110.38688) (end 154.72156 110.98022) (width 0.25) (layer F.Cu) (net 5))
 (segment (start 155.3149 109.17988) (end 155.38806 109.10672) (width 0.25) (layer F.Cu) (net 5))
 (segment (start 155.3149 110.38688) (end 155.3149 109.17988) (width 0.25) (layer F.Cu) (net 5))
 (segment (start 161.02228 106.12018) (end 161.04616 106.14406) (width 0.25) (layer B.Cu) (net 2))
 (segment (start 159.3149 106.12018) (end 161.02228 106.12018) (width 0.25) (layer B.Cu) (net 2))
 (segment (start 159.3149 107.03356) (end 159.38806 107.10672) (width 0.25) (layer B.Cu) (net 2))
 (segment (start 159.3149 106.12018) (end 159.3149 107.03356) (width 0.25) (layer B.Cu) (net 2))
 (segment (start 158.90684 111.90986) (end 159.53486 111.90986) (width 0.25) (layer F.Cu) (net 3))
 (segment (start 157.3149 110.31792) (end 158.90684 111.90986) (width 0.25) (layer F.Cu) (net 3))
 (segment (start 157.3149 109.17988) (end 157.38806 109.10672) (width 0.25) (layer F.Cu) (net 3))
 (segment (start 157.3149 110.31792) (end 157.3149 109.17988) (width 0.25) (layer F.Cu) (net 3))
 (segment (start 155.95854 104.46156) (end 157.32354 105.82656) (width 0.25) (layer F.Cu) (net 4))
 (segment (start 155.95854 103.67518) (end 155.95854 104.46156) (width 0.25) (layer F.Cu) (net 4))
 (segment (start 157.32354 107.0422) (end 157.38806 107.10672) (width 0.25) (layer F.Cu) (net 4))
 (segment (start 157.32354 105.82656) (end 157.32354 107.0422) (width 0.25) (layer F.Cu) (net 4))
 (segment (start 154.8765 105.37952) (end 155.32354 105.82656) (width 0.25) (layer F.Cu) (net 6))
 (segment (start 154.8765 103.67518) (end 154.8765 105.37952) (width 0.25) (layer F.Cu) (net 6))
 (segment (start 155.32354 107.0422) (end 155.38806 107.10672) (width 0.25) (layer F.Cu) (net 6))
 (segment (start 155.32354 105.82656) (end 155.32354 107.0422) (width 0.25) (layer F.Cu) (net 6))
 (segment (start 159.40532 109.12398) (end 159.38806 109.10672) (width 1) (layer F.Cu) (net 1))
 (segment (start 159.40532 110.6043) (end 159.40532 109.12398) (width 1) (layer F.Cu) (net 1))
 (segment (start 149.880601 110.748659) (end 149.52712 111.10214) (width 0.25) (layer F.Cu) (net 8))
 (segment (start 149.55902 103.76282) (end 149.95906 104.16286) (width 1) (layer F.Cu) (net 13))
 (segment (start 149.55902 102.68716) (end 149.55902 103.76282) (width 1) (layer F.Cu) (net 13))
 (segment (start 146.3256 107.61852) (end 147.3073 106.63682) (width 1) (layer F.Cu) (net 12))
 (segment (start 146.3256 108.05418) (end 146.3256 107.61852) (width 1) (layer F.Cu) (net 12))
 (segment (start 164.49802 107.65282) (end 163.40582 106.56062) (width 1) (layer F.Cu) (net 11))
 (segment (start 164.49802 108.41736) (end 164.49802 107.65282) (width 1) (layer F.Cu) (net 11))
 (segment (start 161.72814 103.8822) (end 161.30778 104.30256) (width 1) (layer F.Cu) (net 10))
 (segment (start 161.72814 102.8852) (end 161.72814 103.8822) (width 1) (layer F.Cu) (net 10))
 (segment (start 149.880601 110.614179) (end 151.38806 109.10672) (width 0.25) (layer F.Cu) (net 8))
 (segment (start 149.880601 110.748659) (end 149.880601 110.614179) (width 0.25) (layer F.Cu) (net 8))
 (segment (start 153.38806 107.10672) (end 151.38806 109.10672) (width 0.25) (layer F.Cu) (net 8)))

